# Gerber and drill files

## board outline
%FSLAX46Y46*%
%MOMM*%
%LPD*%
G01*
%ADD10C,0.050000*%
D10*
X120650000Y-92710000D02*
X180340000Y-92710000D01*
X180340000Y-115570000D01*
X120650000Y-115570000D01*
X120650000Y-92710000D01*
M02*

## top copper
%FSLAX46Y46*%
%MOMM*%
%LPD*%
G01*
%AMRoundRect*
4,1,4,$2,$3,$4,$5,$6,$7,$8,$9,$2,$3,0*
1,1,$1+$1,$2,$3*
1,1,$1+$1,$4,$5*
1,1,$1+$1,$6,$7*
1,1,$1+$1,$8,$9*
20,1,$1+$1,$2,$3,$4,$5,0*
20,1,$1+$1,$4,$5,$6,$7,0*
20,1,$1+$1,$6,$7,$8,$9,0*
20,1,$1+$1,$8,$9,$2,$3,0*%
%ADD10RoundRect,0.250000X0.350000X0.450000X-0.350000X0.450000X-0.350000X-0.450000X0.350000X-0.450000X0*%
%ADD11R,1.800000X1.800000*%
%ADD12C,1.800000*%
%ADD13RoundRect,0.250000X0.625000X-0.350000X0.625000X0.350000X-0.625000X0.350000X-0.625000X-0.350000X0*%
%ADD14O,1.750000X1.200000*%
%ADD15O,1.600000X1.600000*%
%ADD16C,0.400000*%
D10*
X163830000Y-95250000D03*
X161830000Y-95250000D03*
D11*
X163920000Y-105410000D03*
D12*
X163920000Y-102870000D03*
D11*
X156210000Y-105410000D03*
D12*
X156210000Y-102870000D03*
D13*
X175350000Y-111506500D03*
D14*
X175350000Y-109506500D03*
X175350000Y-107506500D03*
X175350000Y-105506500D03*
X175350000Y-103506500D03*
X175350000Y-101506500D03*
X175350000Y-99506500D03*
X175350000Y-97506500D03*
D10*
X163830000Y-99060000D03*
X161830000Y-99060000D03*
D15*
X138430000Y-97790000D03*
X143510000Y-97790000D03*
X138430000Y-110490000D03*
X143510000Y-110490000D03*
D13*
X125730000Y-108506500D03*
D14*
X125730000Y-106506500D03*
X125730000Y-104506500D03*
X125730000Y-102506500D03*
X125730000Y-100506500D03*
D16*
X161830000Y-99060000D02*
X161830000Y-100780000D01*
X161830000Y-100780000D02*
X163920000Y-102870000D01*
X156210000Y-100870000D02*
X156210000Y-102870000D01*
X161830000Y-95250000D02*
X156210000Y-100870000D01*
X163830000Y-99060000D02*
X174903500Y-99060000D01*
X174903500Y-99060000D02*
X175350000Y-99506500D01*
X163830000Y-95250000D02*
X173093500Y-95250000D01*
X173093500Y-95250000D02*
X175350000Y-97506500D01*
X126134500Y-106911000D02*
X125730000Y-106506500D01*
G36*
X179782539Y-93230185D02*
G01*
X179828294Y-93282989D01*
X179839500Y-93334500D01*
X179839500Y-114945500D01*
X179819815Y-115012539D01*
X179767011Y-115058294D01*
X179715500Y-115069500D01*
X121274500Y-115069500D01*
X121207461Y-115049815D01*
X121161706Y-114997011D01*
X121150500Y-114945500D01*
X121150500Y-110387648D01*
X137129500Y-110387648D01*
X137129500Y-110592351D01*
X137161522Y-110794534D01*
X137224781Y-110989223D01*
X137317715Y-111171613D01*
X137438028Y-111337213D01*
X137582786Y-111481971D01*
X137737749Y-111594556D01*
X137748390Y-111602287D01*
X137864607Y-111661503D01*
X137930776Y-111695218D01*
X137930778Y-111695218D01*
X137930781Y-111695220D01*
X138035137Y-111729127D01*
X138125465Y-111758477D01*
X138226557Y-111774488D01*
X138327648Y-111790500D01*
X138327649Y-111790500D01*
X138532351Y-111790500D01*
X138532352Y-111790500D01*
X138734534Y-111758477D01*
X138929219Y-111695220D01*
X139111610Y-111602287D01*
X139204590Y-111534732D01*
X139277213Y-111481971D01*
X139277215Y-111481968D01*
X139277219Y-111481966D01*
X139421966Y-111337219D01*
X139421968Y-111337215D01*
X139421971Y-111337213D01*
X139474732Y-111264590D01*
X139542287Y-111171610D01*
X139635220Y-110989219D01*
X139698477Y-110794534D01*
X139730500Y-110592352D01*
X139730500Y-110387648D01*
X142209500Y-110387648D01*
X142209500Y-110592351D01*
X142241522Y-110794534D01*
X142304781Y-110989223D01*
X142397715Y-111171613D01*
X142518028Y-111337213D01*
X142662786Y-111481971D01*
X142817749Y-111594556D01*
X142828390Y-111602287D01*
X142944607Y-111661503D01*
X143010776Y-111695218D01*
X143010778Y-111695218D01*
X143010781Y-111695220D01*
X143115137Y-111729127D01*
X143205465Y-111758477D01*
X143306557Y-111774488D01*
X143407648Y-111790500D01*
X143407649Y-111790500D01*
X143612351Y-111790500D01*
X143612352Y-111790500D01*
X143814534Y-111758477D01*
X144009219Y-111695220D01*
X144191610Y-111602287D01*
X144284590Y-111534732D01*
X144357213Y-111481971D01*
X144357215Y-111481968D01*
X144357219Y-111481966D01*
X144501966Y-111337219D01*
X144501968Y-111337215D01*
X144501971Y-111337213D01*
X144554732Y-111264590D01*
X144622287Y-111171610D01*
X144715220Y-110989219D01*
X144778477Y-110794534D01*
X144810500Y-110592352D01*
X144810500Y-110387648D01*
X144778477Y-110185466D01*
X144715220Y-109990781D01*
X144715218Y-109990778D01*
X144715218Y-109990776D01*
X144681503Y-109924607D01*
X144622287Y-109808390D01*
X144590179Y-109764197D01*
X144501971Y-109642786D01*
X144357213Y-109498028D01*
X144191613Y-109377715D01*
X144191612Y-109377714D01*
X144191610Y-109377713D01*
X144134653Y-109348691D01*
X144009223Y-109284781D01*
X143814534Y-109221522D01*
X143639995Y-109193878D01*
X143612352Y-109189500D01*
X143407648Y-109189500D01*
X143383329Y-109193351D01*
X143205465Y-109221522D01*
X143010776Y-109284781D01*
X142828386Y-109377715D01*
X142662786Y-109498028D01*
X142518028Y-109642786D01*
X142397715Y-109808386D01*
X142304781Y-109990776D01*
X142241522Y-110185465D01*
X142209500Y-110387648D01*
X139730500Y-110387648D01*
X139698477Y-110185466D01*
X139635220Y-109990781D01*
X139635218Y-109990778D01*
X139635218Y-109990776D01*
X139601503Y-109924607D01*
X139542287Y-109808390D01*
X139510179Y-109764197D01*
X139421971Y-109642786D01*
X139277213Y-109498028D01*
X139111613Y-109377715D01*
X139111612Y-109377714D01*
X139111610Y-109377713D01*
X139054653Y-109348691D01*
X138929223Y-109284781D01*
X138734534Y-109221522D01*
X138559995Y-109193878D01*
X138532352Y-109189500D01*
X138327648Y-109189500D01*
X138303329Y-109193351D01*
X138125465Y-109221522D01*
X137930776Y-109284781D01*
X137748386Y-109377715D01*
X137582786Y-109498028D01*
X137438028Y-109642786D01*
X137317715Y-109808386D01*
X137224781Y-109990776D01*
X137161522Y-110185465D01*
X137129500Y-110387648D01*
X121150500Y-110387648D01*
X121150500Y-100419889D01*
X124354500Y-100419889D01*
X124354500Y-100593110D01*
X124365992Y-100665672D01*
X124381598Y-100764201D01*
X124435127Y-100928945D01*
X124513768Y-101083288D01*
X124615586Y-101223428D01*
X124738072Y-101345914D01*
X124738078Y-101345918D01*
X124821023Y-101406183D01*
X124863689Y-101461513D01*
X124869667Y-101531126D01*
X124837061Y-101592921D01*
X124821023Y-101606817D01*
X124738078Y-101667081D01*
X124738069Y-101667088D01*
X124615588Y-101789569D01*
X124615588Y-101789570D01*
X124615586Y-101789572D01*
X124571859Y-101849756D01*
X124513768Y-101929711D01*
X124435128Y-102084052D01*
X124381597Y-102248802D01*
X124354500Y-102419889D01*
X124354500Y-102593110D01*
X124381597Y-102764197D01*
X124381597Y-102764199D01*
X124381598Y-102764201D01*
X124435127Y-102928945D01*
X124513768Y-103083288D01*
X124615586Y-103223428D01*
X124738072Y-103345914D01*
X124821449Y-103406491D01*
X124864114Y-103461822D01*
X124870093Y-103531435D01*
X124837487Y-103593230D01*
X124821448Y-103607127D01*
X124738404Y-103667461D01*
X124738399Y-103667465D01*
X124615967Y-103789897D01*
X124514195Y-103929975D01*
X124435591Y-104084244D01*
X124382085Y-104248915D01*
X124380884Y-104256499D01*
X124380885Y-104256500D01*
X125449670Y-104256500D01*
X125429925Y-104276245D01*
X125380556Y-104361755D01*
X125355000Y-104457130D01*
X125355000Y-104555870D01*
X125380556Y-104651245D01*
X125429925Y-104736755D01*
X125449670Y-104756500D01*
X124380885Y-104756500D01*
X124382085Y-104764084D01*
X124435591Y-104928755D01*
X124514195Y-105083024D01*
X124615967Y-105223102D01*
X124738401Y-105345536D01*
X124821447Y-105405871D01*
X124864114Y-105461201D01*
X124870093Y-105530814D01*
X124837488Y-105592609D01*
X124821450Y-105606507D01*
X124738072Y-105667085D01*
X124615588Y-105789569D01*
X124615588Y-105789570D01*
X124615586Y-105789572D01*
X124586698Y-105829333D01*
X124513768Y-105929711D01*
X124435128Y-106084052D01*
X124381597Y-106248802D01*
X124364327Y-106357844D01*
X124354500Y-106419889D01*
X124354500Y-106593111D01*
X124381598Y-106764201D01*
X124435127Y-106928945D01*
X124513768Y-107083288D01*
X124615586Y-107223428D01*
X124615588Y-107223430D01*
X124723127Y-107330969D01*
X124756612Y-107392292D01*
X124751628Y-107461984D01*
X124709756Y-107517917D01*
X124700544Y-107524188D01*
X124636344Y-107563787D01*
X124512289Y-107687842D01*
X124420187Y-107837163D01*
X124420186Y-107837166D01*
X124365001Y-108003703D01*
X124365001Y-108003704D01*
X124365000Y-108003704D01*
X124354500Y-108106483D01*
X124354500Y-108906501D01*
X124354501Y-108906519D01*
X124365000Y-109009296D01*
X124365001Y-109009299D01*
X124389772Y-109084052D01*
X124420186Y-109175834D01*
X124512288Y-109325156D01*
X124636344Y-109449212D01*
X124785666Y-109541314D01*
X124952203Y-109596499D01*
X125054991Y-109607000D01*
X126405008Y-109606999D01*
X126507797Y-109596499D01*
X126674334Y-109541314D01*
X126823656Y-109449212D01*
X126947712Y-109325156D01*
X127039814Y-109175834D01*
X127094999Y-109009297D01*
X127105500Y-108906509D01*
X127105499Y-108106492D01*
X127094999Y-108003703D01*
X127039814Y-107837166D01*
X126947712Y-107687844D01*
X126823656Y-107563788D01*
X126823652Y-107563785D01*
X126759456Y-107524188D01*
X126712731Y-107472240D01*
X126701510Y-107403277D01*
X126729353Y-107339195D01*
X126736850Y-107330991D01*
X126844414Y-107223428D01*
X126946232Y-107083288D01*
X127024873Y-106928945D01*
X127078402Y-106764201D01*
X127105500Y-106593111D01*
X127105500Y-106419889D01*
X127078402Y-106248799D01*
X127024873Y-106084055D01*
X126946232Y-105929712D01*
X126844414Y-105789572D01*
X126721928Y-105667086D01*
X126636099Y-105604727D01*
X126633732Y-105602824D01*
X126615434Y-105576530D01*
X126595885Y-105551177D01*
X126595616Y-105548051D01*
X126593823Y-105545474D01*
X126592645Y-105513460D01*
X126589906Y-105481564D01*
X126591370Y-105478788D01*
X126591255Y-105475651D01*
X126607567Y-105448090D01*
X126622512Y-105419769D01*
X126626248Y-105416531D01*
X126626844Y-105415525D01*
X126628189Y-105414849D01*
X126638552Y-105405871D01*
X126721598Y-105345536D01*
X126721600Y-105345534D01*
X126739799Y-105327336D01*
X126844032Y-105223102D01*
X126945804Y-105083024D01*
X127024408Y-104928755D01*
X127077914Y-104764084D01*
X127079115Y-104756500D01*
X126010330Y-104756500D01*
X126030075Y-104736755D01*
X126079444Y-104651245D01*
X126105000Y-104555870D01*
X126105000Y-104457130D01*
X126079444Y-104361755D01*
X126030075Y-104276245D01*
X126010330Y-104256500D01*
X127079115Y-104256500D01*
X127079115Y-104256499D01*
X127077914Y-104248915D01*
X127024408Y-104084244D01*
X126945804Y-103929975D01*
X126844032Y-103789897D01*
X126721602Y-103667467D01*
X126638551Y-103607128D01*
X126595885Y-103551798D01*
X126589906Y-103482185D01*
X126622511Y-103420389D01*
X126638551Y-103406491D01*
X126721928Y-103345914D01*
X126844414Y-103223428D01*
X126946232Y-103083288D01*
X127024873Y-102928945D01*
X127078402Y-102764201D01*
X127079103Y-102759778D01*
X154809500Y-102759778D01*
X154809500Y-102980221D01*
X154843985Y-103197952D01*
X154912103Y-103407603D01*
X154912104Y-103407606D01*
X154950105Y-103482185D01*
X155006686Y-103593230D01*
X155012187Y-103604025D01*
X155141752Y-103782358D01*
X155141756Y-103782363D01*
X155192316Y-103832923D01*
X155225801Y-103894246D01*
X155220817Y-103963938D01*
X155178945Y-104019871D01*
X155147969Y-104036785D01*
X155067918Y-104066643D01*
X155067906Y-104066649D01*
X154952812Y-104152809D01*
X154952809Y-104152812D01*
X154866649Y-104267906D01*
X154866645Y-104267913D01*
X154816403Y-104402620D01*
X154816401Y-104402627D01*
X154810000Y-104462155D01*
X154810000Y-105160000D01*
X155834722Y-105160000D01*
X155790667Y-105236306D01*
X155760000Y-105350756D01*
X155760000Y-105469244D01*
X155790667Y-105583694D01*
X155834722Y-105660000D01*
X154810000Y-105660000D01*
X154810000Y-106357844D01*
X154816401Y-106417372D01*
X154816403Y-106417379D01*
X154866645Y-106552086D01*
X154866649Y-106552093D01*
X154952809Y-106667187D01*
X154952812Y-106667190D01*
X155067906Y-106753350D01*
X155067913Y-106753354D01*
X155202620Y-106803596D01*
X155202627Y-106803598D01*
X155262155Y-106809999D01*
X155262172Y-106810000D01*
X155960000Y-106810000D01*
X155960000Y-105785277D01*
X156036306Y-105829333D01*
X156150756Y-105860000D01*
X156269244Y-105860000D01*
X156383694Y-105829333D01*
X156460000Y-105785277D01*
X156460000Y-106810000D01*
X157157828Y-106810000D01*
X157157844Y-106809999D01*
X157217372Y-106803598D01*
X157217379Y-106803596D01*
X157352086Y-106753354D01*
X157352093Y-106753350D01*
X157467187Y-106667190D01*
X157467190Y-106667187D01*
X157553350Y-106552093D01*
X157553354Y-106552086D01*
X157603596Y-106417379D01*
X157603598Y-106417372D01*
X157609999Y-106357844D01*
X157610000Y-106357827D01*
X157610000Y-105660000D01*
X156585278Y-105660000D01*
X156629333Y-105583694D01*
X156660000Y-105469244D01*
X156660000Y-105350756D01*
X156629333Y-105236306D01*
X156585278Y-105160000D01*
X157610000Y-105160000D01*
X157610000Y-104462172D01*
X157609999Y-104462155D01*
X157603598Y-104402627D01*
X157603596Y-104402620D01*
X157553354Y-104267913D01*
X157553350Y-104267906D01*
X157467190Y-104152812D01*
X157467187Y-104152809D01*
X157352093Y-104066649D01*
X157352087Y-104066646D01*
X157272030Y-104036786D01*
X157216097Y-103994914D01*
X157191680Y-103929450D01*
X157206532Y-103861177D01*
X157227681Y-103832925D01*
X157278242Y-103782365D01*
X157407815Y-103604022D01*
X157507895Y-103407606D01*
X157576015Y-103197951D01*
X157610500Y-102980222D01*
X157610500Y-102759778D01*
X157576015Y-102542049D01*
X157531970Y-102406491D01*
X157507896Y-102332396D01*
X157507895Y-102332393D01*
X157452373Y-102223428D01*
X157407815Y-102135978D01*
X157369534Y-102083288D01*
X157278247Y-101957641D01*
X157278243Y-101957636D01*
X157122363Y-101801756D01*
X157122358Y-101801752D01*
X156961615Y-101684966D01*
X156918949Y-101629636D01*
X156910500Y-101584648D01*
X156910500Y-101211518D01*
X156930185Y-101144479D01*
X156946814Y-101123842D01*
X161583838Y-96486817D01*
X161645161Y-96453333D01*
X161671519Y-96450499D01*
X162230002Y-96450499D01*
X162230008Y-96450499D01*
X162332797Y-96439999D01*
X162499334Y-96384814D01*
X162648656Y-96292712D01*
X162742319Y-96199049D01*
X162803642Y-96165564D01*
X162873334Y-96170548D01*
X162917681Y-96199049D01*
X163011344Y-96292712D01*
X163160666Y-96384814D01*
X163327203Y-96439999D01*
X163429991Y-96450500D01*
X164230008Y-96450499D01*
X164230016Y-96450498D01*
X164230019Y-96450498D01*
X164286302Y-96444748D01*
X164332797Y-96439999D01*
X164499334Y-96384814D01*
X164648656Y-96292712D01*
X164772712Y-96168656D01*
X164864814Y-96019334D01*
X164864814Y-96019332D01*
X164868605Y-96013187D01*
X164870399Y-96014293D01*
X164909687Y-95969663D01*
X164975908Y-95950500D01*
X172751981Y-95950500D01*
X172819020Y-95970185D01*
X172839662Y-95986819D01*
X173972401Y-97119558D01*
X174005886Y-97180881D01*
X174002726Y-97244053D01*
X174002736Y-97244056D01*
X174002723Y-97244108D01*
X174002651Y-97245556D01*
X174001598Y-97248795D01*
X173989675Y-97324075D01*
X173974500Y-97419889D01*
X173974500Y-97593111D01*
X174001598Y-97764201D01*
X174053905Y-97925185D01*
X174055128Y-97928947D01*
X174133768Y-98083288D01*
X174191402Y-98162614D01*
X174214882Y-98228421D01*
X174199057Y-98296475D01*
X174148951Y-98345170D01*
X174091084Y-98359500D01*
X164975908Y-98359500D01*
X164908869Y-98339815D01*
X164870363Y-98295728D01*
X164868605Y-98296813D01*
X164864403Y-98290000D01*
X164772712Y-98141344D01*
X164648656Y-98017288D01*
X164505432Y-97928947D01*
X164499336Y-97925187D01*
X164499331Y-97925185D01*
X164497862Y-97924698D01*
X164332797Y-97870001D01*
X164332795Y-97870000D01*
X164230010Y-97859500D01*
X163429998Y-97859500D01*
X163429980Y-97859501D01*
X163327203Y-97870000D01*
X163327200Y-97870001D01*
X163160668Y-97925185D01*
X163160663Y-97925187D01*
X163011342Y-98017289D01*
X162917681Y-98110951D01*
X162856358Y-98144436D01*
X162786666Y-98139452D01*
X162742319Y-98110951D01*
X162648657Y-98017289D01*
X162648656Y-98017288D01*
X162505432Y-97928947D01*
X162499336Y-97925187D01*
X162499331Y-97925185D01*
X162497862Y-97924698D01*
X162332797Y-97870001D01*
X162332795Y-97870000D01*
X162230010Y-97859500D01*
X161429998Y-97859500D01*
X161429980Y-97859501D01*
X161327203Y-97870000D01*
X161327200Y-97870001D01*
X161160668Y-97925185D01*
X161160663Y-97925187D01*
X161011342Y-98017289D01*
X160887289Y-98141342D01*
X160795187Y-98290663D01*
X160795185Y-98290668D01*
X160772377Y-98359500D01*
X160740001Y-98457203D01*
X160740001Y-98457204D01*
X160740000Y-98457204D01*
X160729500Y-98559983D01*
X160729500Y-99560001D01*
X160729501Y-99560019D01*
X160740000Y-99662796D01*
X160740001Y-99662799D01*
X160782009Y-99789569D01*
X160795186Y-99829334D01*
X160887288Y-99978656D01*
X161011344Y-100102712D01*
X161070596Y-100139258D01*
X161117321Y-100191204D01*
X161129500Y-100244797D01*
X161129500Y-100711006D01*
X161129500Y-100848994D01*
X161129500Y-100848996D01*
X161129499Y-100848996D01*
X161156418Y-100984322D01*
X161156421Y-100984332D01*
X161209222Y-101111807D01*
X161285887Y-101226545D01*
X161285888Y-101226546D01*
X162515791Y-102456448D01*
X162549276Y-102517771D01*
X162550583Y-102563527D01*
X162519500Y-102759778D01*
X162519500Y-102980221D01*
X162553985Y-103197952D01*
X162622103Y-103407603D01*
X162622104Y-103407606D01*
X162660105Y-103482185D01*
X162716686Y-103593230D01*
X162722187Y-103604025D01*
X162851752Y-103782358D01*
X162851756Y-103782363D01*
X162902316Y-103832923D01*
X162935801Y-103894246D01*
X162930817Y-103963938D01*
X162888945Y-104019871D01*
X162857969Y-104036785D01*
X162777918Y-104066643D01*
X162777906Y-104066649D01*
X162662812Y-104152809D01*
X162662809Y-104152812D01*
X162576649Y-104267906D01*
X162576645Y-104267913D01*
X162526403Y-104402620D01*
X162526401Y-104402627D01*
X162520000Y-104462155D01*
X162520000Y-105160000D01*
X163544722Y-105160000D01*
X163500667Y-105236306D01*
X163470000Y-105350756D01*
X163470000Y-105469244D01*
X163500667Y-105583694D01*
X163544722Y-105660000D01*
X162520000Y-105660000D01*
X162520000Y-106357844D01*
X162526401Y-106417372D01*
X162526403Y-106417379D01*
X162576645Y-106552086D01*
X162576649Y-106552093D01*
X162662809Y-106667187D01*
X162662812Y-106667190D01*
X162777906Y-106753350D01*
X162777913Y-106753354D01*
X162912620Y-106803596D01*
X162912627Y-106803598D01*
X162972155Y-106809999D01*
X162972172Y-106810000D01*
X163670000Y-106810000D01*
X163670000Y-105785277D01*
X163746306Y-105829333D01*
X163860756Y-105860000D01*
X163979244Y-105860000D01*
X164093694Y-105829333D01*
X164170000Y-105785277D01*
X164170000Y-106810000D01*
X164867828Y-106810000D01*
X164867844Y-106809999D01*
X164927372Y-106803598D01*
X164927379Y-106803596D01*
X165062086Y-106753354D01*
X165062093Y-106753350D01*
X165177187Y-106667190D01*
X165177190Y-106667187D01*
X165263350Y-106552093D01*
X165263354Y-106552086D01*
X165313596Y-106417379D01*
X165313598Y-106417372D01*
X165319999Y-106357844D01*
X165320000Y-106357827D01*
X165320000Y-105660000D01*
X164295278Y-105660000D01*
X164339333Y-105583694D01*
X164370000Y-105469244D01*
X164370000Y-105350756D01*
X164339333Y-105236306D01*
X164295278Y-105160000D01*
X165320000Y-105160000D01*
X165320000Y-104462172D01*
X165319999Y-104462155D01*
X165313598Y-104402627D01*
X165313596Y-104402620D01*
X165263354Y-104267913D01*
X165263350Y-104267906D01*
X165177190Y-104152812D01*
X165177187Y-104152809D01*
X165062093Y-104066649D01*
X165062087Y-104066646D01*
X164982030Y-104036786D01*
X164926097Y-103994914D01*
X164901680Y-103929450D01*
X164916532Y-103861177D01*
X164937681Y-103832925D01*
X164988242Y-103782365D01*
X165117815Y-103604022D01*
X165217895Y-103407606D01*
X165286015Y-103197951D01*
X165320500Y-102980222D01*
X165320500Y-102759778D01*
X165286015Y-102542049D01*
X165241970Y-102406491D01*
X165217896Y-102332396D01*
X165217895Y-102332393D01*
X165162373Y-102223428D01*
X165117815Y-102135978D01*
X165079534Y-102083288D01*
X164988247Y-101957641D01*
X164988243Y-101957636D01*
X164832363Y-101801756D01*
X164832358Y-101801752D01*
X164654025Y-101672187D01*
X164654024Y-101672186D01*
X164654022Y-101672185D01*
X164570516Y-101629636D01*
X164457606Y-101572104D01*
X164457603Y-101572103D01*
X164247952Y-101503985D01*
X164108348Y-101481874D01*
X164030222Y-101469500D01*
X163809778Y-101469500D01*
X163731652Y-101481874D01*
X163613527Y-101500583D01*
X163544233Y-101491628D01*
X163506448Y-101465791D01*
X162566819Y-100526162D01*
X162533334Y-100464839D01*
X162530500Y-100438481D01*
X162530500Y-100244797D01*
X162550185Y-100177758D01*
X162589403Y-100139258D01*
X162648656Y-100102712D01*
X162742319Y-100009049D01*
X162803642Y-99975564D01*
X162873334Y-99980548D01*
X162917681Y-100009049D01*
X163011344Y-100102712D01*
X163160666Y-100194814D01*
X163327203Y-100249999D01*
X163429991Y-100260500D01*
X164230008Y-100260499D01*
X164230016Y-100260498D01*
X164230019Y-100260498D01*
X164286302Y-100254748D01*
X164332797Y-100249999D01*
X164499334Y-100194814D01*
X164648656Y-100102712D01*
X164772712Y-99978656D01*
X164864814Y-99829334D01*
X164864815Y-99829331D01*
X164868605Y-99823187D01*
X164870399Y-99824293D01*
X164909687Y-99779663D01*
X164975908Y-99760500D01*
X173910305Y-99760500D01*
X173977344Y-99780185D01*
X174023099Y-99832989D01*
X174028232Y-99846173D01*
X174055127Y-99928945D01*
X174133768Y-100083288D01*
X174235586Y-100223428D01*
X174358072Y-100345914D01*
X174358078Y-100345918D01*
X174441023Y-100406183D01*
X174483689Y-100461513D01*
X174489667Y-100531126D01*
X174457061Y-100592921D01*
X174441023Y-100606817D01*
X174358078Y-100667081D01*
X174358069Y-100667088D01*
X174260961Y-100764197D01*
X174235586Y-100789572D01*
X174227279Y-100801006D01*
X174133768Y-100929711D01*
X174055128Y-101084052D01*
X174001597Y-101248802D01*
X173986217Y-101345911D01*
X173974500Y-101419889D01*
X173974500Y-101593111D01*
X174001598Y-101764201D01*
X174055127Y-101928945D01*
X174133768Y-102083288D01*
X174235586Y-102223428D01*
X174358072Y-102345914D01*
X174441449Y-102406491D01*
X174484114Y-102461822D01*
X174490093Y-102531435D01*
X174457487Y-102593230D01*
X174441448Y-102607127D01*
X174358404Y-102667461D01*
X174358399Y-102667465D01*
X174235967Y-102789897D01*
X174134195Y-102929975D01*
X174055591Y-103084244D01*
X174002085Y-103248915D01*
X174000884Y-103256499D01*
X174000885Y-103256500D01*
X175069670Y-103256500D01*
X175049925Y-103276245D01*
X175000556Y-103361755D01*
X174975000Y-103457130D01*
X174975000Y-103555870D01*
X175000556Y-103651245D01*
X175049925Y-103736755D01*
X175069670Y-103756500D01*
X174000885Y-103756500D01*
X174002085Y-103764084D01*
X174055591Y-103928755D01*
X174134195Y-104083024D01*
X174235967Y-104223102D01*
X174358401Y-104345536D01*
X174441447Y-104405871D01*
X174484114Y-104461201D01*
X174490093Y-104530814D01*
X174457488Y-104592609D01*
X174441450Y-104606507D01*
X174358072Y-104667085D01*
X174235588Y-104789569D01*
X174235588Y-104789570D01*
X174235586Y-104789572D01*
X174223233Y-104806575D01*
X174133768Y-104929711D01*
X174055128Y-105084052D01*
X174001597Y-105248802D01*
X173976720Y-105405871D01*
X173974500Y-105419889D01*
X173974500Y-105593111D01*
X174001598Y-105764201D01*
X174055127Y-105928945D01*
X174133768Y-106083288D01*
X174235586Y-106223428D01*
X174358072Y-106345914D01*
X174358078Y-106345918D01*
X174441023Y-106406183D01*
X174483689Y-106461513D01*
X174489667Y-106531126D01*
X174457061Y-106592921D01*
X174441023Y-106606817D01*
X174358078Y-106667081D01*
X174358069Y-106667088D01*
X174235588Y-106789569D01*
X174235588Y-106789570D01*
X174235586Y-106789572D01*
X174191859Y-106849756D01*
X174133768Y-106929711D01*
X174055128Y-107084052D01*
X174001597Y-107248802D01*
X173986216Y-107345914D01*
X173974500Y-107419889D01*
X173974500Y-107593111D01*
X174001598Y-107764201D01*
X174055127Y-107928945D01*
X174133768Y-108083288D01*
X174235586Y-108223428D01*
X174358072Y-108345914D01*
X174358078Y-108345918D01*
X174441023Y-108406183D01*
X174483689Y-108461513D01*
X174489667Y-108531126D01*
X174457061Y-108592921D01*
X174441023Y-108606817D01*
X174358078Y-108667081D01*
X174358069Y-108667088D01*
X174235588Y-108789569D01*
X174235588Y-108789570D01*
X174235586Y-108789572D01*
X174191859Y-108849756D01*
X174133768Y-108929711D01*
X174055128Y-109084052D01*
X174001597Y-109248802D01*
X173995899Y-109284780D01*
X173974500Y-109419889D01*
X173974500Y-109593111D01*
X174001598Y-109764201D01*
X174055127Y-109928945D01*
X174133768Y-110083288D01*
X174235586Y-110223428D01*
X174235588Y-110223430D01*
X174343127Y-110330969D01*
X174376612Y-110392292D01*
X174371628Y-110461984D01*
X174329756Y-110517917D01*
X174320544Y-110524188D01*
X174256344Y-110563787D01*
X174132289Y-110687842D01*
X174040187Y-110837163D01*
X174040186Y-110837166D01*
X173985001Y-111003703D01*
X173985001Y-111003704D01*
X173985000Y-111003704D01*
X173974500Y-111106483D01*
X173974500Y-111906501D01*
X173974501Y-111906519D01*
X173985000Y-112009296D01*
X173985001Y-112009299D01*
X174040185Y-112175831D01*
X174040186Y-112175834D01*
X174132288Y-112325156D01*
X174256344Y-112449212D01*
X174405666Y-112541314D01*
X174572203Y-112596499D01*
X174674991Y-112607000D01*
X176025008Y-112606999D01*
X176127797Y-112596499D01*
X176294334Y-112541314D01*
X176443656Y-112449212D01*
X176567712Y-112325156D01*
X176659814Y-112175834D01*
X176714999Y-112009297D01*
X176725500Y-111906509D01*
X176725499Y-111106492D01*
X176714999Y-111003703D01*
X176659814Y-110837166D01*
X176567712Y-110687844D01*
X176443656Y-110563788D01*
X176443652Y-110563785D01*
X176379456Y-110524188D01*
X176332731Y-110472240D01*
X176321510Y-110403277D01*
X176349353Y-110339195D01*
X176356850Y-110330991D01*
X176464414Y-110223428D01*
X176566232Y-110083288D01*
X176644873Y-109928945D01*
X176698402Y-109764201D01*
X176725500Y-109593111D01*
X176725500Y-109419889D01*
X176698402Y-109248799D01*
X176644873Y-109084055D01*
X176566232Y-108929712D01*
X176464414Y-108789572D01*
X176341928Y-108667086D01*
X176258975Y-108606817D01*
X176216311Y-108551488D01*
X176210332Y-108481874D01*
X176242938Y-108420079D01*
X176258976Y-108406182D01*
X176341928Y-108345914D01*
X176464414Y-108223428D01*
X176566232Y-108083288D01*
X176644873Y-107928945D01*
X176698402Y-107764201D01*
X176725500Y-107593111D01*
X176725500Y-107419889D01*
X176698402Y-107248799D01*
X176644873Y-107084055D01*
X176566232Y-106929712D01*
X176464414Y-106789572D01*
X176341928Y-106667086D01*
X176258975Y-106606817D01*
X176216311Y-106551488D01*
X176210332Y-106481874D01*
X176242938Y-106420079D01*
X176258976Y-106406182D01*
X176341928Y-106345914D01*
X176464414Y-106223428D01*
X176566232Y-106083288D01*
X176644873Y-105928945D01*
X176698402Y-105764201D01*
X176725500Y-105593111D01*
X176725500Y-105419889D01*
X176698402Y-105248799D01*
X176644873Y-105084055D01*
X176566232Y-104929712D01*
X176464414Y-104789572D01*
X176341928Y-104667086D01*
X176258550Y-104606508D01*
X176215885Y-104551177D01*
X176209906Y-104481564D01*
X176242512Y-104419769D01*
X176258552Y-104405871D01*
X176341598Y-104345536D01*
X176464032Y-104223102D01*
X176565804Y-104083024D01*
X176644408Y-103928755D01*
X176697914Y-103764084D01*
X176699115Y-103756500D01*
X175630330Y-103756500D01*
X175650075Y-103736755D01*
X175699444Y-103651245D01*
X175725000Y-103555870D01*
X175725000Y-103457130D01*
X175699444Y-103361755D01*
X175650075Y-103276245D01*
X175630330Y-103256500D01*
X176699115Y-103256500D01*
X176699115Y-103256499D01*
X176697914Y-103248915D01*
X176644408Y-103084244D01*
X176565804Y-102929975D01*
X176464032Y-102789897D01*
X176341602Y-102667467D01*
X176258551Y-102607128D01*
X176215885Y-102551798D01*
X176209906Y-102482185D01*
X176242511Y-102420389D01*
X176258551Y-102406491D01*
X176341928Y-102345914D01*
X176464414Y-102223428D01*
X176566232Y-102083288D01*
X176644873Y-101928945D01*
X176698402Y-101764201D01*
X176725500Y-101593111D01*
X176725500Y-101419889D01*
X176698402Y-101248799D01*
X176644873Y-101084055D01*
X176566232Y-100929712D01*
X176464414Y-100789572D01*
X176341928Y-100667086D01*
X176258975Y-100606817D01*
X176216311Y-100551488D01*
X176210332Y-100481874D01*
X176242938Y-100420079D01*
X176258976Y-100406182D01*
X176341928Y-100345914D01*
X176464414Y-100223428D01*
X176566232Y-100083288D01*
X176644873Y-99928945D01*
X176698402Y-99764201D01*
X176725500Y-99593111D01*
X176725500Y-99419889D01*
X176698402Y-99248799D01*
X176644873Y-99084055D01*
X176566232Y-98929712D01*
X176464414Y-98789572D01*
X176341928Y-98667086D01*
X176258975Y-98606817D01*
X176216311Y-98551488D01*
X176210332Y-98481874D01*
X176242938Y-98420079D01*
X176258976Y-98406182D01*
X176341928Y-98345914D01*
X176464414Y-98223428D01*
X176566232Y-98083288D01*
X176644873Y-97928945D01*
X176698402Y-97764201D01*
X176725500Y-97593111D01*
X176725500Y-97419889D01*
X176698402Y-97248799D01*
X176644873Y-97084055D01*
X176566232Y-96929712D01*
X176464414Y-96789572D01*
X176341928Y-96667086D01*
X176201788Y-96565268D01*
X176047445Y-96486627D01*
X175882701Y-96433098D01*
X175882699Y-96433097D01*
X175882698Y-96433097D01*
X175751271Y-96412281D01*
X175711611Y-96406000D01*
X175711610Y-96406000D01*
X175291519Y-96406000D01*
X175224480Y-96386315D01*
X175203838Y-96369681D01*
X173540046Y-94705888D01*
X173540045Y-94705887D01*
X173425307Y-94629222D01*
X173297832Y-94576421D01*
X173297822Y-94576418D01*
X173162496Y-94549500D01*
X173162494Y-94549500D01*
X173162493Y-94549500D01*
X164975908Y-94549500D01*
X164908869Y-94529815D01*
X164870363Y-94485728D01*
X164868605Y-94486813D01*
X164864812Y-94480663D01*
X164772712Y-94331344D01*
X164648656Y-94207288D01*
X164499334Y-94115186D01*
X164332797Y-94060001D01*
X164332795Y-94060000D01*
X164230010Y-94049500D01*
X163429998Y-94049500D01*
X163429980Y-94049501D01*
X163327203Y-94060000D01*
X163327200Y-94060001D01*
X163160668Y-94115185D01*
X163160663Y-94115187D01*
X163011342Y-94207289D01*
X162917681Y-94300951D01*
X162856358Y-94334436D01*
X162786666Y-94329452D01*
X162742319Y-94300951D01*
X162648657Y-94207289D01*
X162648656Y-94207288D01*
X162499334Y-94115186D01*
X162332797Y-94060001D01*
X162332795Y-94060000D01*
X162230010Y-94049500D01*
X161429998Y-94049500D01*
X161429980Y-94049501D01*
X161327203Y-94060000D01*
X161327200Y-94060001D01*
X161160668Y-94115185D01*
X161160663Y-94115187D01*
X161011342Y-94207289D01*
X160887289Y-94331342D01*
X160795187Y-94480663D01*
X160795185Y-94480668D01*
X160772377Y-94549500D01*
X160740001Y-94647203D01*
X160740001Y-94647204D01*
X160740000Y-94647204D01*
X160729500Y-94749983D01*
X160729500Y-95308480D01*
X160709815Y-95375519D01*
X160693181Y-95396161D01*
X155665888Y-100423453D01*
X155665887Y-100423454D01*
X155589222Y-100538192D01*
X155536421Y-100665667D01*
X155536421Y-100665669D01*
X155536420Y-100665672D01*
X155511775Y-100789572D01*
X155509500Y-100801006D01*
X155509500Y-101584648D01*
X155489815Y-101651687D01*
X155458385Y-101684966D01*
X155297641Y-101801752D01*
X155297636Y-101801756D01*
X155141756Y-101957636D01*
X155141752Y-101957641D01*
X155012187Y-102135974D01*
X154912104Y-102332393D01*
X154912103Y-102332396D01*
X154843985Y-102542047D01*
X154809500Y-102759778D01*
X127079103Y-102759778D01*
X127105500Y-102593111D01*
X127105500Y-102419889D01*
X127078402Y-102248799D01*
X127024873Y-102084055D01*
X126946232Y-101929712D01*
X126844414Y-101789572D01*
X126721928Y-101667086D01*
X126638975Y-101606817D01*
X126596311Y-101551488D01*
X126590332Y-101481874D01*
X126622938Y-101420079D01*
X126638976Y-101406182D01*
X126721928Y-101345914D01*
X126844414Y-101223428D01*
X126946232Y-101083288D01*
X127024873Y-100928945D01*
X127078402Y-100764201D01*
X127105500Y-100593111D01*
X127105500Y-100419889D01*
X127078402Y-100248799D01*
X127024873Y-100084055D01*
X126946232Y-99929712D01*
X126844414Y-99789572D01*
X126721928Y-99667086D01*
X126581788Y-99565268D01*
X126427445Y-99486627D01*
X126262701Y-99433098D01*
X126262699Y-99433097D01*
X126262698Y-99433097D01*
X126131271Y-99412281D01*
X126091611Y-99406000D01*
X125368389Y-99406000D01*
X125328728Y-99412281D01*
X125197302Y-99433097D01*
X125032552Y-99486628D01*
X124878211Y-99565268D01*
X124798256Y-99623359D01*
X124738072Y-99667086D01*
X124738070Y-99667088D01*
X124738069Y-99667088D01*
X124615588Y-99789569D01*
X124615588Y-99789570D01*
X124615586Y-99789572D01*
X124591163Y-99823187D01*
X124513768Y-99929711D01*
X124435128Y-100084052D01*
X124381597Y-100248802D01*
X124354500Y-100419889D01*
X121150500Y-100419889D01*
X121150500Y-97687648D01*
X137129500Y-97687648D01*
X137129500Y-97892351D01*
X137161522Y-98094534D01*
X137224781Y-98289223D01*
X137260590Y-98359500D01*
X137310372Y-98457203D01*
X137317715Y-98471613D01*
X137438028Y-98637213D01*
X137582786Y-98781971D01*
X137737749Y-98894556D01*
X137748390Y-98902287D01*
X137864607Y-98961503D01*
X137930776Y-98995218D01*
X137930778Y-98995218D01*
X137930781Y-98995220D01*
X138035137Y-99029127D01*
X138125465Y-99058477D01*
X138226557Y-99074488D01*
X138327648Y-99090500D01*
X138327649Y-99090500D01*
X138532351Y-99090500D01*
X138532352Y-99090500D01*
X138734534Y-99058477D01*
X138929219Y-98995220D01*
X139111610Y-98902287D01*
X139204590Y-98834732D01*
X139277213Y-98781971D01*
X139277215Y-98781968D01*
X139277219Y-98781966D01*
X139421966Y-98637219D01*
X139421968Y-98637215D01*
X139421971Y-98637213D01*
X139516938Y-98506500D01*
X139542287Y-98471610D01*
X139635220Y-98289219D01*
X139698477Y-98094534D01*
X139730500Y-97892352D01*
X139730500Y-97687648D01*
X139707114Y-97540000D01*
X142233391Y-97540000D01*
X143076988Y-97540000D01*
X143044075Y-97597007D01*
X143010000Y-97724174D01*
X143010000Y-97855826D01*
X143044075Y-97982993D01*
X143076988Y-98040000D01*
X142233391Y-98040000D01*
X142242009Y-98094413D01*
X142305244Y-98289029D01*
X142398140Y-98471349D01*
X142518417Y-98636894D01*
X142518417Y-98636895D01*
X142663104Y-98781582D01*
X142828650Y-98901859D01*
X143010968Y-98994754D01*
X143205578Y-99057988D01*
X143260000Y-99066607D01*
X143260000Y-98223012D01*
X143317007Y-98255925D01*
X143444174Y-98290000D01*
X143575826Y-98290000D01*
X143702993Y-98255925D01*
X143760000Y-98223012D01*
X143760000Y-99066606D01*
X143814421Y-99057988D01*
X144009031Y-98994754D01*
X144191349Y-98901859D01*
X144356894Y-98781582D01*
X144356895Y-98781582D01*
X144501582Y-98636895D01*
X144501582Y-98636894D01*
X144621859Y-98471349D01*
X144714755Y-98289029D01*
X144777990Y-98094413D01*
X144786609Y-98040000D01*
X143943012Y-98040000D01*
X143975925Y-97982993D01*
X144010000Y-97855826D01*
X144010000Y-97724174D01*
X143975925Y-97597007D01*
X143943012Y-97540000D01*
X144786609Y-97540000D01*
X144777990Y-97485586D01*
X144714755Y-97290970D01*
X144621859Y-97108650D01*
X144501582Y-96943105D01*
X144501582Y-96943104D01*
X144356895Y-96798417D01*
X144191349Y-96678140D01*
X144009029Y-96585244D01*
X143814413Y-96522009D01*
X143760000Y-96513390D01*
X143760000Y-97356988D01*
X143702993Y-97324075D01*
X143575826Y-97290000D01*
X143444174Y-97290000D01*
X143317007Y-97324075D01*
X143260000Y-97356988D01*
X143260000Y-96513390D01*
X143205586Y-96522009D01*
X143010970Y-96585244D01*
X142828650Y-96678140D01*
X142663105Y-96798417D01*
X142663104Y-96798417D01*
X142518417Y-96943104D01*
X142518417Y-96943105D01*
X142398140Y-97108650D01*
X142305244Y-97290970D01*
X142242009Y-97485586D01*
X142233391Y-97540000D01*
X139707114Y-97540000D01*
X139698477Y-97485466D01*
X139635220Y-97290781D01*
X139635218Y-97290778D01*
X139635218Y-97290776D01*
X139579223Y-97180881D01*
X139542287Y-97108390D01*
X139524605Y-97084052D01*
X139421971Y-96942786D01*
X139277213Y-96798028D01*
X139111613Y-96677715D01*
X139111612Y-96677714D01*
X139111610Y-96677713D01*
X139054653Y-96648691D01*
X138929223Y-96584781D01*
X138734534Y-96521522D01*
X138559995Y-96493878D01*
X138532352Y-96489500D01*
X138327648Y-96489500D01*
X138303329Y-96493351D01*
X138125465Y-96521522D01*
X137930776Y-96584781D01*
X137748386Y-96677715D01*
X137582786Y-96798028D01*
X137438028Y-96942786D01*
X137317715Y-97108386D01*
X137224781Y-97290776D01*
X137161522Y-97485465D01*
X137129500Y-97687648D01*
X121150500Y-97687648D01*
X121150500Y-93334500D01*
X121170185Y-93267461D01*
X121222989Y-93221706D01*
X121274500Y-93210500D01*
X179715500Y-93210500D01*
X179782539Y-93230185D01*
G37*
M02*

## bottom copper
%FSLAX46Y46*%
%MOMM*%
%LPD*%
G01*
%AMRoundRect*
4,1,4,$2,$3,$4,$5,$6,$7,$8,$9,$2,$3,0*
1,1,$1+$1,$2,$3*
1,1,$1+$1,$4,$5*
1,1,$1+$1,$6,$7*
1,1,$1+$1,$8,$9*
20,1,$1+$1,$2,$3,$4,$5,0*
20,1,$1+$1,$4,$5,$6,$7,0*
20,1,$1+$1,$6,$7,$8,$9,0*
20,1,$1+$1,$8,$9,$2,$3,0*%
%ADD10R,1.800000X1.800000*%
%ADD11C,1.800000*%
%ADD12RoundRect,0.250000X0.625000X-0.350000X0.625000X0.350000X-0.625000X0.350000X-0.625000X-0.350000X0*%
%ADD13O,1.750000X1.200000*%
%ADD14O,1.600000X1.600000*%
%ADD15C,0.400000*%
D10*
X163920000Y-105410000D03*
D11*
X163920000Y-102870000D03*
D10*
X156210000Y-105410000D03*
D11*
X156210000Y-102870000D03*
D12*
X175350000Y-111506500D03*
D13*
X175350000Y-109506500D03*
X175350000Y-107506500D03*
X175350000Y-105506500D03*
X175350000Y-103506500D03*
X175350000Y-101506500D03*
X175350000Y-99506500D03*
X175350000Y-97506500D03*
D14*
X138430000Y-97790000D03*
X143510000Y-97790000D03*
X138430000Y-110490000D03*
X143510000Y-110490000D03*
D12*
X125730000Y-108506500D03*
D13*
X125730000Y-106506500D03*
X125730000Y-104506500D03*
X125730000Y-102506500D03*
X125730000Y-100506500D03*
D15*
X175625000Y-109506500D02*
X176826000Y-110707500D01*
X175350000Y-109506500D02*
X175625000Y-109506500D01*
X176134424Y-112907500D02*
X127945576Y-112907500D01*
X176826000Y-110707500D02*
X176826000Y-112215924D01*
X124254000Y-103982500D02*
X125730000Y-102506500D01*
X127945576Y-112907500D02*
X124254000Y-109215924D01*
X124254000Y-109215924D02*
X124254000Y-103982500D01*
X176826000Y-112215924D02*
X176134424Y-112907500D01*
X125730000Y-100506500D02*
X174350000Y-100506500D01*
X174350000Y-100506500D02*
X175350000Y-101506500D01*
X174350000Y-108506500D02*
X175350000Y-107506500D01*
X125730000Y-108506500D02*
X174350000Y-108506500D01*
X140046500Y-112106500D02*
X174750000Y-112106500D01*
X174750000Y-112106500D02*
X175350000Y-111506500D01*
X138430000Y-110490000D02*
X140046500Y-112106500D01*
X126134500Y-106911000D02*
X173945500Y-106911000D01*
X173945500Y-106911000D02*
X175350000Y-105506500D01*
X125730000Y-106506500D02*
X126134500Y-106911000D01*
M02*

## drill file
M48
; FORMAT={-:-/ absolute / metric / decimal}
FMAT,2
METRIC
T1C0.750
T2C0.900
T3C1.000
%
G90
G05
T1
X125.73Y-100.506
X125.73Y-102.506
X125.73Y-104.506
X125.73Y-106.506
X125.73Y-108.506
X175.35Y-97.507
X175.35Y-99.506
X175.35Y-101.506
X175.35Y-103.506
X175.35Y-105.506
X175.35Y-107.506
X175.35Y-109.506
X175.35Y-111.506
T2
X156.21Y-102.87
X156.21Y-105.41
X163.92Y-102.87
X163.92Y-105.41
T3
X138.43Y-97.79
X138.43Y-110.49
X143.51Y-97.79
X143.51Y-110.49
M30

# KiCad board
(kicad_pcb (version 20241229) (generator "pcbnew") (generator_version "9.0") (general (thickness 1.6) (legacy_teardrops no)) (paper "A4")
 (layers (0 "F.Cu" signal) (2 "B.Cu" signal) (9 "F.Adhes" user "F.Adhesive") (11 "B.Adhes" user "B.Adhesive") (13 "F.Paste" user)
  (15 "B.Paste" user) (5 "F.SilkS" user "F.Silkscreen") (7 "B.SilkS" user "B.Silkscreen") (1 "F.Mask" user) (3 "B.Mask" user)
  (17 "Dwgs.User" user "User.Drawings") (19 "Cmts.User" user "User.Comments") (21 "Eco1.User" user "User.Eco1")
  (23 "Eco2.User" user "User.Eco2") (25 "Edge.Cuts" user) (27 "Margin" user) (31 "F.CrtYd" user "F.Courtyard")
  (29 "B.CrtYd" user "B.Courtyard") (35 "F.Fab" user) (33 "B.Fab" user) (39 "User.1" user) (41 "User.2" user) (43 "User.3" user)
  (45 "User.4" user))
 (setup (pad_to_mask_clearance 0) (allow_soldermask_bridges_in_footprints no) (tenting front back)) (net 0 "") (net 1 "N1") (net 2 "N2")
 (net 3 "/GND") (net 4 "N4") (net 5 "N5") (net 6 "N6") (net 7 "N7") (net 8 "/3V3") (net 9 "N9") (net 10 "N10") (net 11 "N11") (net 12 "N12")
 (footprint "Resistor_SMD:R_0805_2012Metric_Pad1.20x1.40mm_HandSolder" (layer "F.Cu") (at 162.83 95.25 180)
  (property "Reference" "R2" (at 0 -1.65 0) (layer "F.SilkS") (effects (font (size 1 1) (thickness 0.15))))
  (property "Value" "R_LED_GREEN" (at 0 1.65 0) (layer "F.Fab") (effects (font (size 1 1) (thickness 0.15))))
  (pad "1" smd roundrect (at -1 0 180) (size 1.2 1.4) (layers "F.Cu" "F.Mask" "F.Paste") (roundrect_rratio 0.208333) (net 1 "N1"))
  (pad "2" smd roundrect (at 1 0 180) (size 1.2 1.4) (layers "F.Cu" "F.Mask" "F.Paste") (roundrect_rratio 0.208333) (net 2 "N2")))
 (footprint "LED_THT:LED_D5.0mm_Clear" (layer "F.Cu") (at 163.92 105.41 90)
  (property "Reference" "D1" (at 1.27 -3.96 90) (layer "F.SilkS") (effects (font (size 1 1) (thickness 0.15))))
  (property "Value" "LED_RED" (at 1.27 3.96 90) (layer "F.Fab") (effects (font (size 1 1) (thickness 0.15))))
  (pad "1" thru_hole rect (at 0 0 90) (size 1.8 1.8) (drill 0.9) (layers "*.Cu" "*.Mask") (remove_unused_layers no) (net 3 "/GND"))
  (pad "2" thru_hole circle (at 2.54 0 90) (size 1.8 1.8) (drill 0.9) (layers "*.Cu" "*.Mask") (remove_unused_layers no) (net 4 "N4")))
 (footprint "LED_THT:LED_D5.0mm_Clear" (layer "F.Cu") (at 156.21 105.41 90)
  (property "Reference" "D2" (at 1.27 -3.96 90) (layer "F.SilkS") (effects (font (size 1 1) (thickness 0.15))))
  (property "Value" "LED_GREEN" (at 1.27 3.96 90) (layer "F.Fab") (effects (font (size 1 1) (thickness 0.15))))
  (pad "1" thru_hole rect (at 0 0 90) (size 1.8 1.8) (drill 0.9) (layers "*.Cu" "*.Mask") (remove_unused_layers no) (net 3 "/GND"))
  (pad "2" thru_hole circle (at 2.54 0 90) (size 1.8 1.8) (drill 0.9) (layers "*.Cu" "*.Mask") (remove_unused_layers no) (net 2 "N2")))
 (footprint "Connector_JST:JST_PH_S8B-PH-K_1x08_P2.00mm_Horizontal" (layer "F.Cu") (at 175.35 111.5065 90)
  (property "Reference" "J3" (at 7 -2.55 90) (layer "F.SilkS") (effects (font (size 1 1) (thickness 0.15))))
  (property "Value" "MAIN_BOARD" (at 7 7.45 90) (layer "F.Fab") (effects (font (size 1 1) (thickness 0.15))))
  (pad "1" thru_hole roundrect (at 0 0 90) (size 1.2 1.75) (drill 0.75) (layers "*.Cu" "*.Mask") (remove_unused_layers no)
   (roundrect_rratio 0.208333) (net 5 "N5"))
  (pad "2" thru_hole oval (at 2 0 90) (size 1.2 1.75) (drill 0.75) (layers "*.Cu" "*.Mask") (remove_unused_layers no) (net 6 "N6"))
  (pad "3" thru_hole oval (at 4 0 90) (size 1.2 1.75) (drill 0.75) (layers "*.Cu" "*.Mask") (remove_unused_layers no) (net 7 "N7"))
  (pad "4" thru_hole oval (at 6 0 90) (size 1.2 1.75) (drill 0.75) (layers "*.Cu" "*.Mask") (remove_unused_layers no) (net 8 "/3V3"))
  (pad "5" thru_hole oval (at 8 0 90) (size 1.2 1.75) (drill 0.75) (layers "*.Cu" "*.Mask") (remove_unused_layers no) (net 3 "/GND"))
  (pad "6" thru_hole oval (at 10 0 90) (size 1.2 1.75) (drill 0.75) (layers "*.Cu" "*.Mask") (remove_unused_layers no) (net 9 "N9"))
  (pad "7" thru_hole oval (at 12 0 90) (size 1.2 1.75) (drill 0.75) (layers "*.Cu" "*.Mask") (remove_unused_layers no) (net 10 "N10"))
  (pad "8" thru_hole oval (at 14 0 90) (size 1.2 1.75) (drill 0.75) (layers "*.Cu" "*.Mask") (remove_unused_layers no) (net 1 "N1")))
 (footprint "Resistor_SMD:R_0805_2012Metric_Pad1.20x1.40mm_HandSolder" (layer "F.Cu") (at 162.83 99.06 180)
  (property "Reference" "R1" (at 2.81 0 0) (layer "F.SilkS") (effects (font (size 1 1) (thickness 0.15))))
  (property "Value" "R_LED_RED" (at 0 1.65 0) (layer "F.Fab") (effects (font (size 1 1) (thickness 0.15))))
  (pad "1" smd roundrect (at -1 0 180) (size 1.2 1.4) (layers "F.Cu" "F.Mask" "F.Paste") (roundrect_rratio 0.208333) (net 10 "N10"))
  (pad "2" smd roundrect (at 1 0 180) (size 1.2 1.4) (layers "F.Cu" "F.Mask" "F.Paste") (roundrect_rratio 0.208333) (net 4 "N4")))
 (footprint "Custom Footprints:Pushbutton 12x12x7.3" (layer "F.Cu") (at 140.97 112.395)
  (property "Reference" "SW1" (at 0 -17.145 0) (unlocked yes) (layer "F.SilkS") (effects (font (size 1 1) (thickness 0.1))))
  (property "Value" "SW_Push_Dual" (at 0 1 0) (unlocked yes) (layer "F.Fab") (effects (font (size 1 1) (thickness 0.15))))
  (pad "1" thru_hole oval (at -2.54 -14.605) (size 1.6 1.6) (drill 1) (layers "*.Cu" "*.Mask") (remove_unused_layers no) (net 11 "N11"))
  (pad "2" thru_hole oval (at 2.54 -14.605) (size 1.6 1.6) (drill 1) (layers "*.Cu" "*.Mask") (remove_unused_layers no) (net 3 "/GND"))
  (pad "3" thru_hole oval (at -2.54 -1.905) (size 1.6 1.6) (drill 1) (layers "*.Cu" "*.Mask") (remove_unused_layers no) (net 5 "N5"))
  (pad "4" thru_hole oval (at 2.54 -1.905) (size 1.6 1.6) (drill 1) (layers "*.Cu" "*.Mask") (remove_unused_layers no) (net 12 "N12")))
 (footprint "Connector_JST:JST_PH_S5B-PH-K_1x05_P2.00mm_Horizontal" (layer "B.Cu") (at 125.73 108.5065 90)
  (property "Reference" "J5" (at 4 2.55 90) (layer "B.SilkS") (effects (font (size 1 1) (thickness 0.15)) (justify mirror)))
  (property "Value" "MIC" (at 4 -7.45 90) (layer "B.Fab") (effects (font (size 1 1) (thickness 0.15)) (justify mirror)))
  (pad "1" thru_hole roundrect (at 0 0 90) (size 1.2 1.75) (drill 0.75) (layers "*.Cu" "*.Mask") (remove_unused_layers no)
   (roundrect_rratio 0.208333) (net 7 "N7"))
  (pad "2" thru_hole oval (at 2 0 90) (size 1.2 1.75) (drill 0.75) (layers "*.Cu" "*.Mask") (remove_unused_layers no) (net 8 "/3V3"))
  (pad "3" thru_hole oval (at 4 0 90) (size 1.2 1.75) (drill 0.75) (layers "*.Cu" "*.Mask") (remove_unused_layers no) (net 3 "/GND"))
  (pad "4" thru_hole oval (at 6 0 90) (size 1.2 1.75) (drill 0.75) (layers "*.Cu" "*.Mask") (remove_unused_layers no) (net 6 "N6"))
  (pad "5" thru_hole oval (at 8 0 90) (size 1.2 1.75) (drill 0.75) (layers "*.Cu" "*.Mask") (remove_unused_layers no) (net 9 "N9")))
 (gr_rect (start 120.65 92.71) (end 180.34 115.57) (stroke (width 0.05) (type default)) (fill no) (layer "Edge.Cuts"))
 (segment (start 161.83 99.06) (end 161.83 100.78) (width 0.4) (layer "F.Cu") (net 4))
 (segment (start 161.83 100.78) (end 163.92 102.87) (width 0.4) (layer "F.Cu") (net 4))
 (segment (start 156.21 100.87) (end 156.21 102.87) (width 0.4) (layer "F.Cu") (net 2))
 (segment (start 161.83 95.25) (end 156.21 100.87) (width 0.4) (layer "F.Cu") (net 2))
 (segment (start 175.625 109.5065) (end 176.826 110.7075) (width 0.4) (layer "B.Cu") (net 6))
 (segment (start 175.35 109.5065) (end 175.625 109.5065) (width 0.4) (layer "B.Cu") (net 6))
 (segment (start 176.134424 112.9075) (end 127.945576 112.9075) (width 0.4) (layer "B.Cu") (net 6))
 (segment (start 176.826 110.7075) (end 176.826 112.215924) (width 0.4) (layer "B.Cu") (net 6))
 (segment (start 124.254 103.9825) (end 125.73 102.5065) (width 0.4) (layer "B.Cu") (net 6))
 (segment (start 127.945576 112.9075) (end 124.254 109.215924) (width 0.4) (layer "B.Cu") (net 6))
 (segment (start 124.254 109.215924) (end 124.254 103.9825) (width 0.4) (layer "B.Cu") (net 6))
 (segment (start 176.826 112.215924) (end 176.134424 112.9075) (width 0.4) (layer "B.Cu") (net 6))
 (segment (start 163.83 99.06) (end 174.9035 99.06) (width 0.4) (layer "F.Cu") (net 10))
 (segment (start 174.9035 99.06) (end 175.35 99.5065) (width 0.4) (layer "F.Cu") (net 10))
 (segment (start 125.73 100.5065) (end 174.35 100.5065) (width 0.4) (layer "B.Cu") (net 9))
 (segment (start 174.35 100.5065) (end 175.35 101.5065) (width 0.4) (layer "B.Cu") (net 9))
 (segment (start 163.83 95.25) (end 173.0935 95.25) (width 0.4) (layer "F.Cu") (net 1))
 (segment (start 173.0935 95.25) (end 175.35 97.5065) (width 0.4) (layer "F.Cu") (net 1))
 (segment (start 174.35 108.5065) (end 175.35 107.5065) (width 0.4) (layer "B.Cu") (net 7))
 (segment (start 125.73 108.5065) (end 174.35 108.5065) (width 0.4) (layer "B.Cu") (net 7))
 (segment (start 140.0465 112.1065) (end 174.75 112.1065) (width 0.4) (layer "B.Cu") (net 5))
 (segment (start 174.75 112.1065) (end 175.35 111.5065) (width 0.4) (layer "B.Cu") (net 5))
 (segment (start 138.43 110.49) (end 140.0465 112.1065) (width 0.4) (layer "B.Cu") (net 5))
 (segment (start 126.1345 106.911) (end 125.73 106.5065) (width 0.4) (layer "F.Cu") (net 8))
 (segment (start 126.1345 106.911) (end 173.9455 106.911) (width 0.4) (layer "B.Cu") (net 8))
 (segment (start 173.9455 106.911) (end 175.35 105.5065) (width 0.4) (layer "B.Cu") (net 8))
 (segment (start 125.73 106.5065) (end 126.1345 106.911) (width 0.4) (layer "B.Cu") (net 8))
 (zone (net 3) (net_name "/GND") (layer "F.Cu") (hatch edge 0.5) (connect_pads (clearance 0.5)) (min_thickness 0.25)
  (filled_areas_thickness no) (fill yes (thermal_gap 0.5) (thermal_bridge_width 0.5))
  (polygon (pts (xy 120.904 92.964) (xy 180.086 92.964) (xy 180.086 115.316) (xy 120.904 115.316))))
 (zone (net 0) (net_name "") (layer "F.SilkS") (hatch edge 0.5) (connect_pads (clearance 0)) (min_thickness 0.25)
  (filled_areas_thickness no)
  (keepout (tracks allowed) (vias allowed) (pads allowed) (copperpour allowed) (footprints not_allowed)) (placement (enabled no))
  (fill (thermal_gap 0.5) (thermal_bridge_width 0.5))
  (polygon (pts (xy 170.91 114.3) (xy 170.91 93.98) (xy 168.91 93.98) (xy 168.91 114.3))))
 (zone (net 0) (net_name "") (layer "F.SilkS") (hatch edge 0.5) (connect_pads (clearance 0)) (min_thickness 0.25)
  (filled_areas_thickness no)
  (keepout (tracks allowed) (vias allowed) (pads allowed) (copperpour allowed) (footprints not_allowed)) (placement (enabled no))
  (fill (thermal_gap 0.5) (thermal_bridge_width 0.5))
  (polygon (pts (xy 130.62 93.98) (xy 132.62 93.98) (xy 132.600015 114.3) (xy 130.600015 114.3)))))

